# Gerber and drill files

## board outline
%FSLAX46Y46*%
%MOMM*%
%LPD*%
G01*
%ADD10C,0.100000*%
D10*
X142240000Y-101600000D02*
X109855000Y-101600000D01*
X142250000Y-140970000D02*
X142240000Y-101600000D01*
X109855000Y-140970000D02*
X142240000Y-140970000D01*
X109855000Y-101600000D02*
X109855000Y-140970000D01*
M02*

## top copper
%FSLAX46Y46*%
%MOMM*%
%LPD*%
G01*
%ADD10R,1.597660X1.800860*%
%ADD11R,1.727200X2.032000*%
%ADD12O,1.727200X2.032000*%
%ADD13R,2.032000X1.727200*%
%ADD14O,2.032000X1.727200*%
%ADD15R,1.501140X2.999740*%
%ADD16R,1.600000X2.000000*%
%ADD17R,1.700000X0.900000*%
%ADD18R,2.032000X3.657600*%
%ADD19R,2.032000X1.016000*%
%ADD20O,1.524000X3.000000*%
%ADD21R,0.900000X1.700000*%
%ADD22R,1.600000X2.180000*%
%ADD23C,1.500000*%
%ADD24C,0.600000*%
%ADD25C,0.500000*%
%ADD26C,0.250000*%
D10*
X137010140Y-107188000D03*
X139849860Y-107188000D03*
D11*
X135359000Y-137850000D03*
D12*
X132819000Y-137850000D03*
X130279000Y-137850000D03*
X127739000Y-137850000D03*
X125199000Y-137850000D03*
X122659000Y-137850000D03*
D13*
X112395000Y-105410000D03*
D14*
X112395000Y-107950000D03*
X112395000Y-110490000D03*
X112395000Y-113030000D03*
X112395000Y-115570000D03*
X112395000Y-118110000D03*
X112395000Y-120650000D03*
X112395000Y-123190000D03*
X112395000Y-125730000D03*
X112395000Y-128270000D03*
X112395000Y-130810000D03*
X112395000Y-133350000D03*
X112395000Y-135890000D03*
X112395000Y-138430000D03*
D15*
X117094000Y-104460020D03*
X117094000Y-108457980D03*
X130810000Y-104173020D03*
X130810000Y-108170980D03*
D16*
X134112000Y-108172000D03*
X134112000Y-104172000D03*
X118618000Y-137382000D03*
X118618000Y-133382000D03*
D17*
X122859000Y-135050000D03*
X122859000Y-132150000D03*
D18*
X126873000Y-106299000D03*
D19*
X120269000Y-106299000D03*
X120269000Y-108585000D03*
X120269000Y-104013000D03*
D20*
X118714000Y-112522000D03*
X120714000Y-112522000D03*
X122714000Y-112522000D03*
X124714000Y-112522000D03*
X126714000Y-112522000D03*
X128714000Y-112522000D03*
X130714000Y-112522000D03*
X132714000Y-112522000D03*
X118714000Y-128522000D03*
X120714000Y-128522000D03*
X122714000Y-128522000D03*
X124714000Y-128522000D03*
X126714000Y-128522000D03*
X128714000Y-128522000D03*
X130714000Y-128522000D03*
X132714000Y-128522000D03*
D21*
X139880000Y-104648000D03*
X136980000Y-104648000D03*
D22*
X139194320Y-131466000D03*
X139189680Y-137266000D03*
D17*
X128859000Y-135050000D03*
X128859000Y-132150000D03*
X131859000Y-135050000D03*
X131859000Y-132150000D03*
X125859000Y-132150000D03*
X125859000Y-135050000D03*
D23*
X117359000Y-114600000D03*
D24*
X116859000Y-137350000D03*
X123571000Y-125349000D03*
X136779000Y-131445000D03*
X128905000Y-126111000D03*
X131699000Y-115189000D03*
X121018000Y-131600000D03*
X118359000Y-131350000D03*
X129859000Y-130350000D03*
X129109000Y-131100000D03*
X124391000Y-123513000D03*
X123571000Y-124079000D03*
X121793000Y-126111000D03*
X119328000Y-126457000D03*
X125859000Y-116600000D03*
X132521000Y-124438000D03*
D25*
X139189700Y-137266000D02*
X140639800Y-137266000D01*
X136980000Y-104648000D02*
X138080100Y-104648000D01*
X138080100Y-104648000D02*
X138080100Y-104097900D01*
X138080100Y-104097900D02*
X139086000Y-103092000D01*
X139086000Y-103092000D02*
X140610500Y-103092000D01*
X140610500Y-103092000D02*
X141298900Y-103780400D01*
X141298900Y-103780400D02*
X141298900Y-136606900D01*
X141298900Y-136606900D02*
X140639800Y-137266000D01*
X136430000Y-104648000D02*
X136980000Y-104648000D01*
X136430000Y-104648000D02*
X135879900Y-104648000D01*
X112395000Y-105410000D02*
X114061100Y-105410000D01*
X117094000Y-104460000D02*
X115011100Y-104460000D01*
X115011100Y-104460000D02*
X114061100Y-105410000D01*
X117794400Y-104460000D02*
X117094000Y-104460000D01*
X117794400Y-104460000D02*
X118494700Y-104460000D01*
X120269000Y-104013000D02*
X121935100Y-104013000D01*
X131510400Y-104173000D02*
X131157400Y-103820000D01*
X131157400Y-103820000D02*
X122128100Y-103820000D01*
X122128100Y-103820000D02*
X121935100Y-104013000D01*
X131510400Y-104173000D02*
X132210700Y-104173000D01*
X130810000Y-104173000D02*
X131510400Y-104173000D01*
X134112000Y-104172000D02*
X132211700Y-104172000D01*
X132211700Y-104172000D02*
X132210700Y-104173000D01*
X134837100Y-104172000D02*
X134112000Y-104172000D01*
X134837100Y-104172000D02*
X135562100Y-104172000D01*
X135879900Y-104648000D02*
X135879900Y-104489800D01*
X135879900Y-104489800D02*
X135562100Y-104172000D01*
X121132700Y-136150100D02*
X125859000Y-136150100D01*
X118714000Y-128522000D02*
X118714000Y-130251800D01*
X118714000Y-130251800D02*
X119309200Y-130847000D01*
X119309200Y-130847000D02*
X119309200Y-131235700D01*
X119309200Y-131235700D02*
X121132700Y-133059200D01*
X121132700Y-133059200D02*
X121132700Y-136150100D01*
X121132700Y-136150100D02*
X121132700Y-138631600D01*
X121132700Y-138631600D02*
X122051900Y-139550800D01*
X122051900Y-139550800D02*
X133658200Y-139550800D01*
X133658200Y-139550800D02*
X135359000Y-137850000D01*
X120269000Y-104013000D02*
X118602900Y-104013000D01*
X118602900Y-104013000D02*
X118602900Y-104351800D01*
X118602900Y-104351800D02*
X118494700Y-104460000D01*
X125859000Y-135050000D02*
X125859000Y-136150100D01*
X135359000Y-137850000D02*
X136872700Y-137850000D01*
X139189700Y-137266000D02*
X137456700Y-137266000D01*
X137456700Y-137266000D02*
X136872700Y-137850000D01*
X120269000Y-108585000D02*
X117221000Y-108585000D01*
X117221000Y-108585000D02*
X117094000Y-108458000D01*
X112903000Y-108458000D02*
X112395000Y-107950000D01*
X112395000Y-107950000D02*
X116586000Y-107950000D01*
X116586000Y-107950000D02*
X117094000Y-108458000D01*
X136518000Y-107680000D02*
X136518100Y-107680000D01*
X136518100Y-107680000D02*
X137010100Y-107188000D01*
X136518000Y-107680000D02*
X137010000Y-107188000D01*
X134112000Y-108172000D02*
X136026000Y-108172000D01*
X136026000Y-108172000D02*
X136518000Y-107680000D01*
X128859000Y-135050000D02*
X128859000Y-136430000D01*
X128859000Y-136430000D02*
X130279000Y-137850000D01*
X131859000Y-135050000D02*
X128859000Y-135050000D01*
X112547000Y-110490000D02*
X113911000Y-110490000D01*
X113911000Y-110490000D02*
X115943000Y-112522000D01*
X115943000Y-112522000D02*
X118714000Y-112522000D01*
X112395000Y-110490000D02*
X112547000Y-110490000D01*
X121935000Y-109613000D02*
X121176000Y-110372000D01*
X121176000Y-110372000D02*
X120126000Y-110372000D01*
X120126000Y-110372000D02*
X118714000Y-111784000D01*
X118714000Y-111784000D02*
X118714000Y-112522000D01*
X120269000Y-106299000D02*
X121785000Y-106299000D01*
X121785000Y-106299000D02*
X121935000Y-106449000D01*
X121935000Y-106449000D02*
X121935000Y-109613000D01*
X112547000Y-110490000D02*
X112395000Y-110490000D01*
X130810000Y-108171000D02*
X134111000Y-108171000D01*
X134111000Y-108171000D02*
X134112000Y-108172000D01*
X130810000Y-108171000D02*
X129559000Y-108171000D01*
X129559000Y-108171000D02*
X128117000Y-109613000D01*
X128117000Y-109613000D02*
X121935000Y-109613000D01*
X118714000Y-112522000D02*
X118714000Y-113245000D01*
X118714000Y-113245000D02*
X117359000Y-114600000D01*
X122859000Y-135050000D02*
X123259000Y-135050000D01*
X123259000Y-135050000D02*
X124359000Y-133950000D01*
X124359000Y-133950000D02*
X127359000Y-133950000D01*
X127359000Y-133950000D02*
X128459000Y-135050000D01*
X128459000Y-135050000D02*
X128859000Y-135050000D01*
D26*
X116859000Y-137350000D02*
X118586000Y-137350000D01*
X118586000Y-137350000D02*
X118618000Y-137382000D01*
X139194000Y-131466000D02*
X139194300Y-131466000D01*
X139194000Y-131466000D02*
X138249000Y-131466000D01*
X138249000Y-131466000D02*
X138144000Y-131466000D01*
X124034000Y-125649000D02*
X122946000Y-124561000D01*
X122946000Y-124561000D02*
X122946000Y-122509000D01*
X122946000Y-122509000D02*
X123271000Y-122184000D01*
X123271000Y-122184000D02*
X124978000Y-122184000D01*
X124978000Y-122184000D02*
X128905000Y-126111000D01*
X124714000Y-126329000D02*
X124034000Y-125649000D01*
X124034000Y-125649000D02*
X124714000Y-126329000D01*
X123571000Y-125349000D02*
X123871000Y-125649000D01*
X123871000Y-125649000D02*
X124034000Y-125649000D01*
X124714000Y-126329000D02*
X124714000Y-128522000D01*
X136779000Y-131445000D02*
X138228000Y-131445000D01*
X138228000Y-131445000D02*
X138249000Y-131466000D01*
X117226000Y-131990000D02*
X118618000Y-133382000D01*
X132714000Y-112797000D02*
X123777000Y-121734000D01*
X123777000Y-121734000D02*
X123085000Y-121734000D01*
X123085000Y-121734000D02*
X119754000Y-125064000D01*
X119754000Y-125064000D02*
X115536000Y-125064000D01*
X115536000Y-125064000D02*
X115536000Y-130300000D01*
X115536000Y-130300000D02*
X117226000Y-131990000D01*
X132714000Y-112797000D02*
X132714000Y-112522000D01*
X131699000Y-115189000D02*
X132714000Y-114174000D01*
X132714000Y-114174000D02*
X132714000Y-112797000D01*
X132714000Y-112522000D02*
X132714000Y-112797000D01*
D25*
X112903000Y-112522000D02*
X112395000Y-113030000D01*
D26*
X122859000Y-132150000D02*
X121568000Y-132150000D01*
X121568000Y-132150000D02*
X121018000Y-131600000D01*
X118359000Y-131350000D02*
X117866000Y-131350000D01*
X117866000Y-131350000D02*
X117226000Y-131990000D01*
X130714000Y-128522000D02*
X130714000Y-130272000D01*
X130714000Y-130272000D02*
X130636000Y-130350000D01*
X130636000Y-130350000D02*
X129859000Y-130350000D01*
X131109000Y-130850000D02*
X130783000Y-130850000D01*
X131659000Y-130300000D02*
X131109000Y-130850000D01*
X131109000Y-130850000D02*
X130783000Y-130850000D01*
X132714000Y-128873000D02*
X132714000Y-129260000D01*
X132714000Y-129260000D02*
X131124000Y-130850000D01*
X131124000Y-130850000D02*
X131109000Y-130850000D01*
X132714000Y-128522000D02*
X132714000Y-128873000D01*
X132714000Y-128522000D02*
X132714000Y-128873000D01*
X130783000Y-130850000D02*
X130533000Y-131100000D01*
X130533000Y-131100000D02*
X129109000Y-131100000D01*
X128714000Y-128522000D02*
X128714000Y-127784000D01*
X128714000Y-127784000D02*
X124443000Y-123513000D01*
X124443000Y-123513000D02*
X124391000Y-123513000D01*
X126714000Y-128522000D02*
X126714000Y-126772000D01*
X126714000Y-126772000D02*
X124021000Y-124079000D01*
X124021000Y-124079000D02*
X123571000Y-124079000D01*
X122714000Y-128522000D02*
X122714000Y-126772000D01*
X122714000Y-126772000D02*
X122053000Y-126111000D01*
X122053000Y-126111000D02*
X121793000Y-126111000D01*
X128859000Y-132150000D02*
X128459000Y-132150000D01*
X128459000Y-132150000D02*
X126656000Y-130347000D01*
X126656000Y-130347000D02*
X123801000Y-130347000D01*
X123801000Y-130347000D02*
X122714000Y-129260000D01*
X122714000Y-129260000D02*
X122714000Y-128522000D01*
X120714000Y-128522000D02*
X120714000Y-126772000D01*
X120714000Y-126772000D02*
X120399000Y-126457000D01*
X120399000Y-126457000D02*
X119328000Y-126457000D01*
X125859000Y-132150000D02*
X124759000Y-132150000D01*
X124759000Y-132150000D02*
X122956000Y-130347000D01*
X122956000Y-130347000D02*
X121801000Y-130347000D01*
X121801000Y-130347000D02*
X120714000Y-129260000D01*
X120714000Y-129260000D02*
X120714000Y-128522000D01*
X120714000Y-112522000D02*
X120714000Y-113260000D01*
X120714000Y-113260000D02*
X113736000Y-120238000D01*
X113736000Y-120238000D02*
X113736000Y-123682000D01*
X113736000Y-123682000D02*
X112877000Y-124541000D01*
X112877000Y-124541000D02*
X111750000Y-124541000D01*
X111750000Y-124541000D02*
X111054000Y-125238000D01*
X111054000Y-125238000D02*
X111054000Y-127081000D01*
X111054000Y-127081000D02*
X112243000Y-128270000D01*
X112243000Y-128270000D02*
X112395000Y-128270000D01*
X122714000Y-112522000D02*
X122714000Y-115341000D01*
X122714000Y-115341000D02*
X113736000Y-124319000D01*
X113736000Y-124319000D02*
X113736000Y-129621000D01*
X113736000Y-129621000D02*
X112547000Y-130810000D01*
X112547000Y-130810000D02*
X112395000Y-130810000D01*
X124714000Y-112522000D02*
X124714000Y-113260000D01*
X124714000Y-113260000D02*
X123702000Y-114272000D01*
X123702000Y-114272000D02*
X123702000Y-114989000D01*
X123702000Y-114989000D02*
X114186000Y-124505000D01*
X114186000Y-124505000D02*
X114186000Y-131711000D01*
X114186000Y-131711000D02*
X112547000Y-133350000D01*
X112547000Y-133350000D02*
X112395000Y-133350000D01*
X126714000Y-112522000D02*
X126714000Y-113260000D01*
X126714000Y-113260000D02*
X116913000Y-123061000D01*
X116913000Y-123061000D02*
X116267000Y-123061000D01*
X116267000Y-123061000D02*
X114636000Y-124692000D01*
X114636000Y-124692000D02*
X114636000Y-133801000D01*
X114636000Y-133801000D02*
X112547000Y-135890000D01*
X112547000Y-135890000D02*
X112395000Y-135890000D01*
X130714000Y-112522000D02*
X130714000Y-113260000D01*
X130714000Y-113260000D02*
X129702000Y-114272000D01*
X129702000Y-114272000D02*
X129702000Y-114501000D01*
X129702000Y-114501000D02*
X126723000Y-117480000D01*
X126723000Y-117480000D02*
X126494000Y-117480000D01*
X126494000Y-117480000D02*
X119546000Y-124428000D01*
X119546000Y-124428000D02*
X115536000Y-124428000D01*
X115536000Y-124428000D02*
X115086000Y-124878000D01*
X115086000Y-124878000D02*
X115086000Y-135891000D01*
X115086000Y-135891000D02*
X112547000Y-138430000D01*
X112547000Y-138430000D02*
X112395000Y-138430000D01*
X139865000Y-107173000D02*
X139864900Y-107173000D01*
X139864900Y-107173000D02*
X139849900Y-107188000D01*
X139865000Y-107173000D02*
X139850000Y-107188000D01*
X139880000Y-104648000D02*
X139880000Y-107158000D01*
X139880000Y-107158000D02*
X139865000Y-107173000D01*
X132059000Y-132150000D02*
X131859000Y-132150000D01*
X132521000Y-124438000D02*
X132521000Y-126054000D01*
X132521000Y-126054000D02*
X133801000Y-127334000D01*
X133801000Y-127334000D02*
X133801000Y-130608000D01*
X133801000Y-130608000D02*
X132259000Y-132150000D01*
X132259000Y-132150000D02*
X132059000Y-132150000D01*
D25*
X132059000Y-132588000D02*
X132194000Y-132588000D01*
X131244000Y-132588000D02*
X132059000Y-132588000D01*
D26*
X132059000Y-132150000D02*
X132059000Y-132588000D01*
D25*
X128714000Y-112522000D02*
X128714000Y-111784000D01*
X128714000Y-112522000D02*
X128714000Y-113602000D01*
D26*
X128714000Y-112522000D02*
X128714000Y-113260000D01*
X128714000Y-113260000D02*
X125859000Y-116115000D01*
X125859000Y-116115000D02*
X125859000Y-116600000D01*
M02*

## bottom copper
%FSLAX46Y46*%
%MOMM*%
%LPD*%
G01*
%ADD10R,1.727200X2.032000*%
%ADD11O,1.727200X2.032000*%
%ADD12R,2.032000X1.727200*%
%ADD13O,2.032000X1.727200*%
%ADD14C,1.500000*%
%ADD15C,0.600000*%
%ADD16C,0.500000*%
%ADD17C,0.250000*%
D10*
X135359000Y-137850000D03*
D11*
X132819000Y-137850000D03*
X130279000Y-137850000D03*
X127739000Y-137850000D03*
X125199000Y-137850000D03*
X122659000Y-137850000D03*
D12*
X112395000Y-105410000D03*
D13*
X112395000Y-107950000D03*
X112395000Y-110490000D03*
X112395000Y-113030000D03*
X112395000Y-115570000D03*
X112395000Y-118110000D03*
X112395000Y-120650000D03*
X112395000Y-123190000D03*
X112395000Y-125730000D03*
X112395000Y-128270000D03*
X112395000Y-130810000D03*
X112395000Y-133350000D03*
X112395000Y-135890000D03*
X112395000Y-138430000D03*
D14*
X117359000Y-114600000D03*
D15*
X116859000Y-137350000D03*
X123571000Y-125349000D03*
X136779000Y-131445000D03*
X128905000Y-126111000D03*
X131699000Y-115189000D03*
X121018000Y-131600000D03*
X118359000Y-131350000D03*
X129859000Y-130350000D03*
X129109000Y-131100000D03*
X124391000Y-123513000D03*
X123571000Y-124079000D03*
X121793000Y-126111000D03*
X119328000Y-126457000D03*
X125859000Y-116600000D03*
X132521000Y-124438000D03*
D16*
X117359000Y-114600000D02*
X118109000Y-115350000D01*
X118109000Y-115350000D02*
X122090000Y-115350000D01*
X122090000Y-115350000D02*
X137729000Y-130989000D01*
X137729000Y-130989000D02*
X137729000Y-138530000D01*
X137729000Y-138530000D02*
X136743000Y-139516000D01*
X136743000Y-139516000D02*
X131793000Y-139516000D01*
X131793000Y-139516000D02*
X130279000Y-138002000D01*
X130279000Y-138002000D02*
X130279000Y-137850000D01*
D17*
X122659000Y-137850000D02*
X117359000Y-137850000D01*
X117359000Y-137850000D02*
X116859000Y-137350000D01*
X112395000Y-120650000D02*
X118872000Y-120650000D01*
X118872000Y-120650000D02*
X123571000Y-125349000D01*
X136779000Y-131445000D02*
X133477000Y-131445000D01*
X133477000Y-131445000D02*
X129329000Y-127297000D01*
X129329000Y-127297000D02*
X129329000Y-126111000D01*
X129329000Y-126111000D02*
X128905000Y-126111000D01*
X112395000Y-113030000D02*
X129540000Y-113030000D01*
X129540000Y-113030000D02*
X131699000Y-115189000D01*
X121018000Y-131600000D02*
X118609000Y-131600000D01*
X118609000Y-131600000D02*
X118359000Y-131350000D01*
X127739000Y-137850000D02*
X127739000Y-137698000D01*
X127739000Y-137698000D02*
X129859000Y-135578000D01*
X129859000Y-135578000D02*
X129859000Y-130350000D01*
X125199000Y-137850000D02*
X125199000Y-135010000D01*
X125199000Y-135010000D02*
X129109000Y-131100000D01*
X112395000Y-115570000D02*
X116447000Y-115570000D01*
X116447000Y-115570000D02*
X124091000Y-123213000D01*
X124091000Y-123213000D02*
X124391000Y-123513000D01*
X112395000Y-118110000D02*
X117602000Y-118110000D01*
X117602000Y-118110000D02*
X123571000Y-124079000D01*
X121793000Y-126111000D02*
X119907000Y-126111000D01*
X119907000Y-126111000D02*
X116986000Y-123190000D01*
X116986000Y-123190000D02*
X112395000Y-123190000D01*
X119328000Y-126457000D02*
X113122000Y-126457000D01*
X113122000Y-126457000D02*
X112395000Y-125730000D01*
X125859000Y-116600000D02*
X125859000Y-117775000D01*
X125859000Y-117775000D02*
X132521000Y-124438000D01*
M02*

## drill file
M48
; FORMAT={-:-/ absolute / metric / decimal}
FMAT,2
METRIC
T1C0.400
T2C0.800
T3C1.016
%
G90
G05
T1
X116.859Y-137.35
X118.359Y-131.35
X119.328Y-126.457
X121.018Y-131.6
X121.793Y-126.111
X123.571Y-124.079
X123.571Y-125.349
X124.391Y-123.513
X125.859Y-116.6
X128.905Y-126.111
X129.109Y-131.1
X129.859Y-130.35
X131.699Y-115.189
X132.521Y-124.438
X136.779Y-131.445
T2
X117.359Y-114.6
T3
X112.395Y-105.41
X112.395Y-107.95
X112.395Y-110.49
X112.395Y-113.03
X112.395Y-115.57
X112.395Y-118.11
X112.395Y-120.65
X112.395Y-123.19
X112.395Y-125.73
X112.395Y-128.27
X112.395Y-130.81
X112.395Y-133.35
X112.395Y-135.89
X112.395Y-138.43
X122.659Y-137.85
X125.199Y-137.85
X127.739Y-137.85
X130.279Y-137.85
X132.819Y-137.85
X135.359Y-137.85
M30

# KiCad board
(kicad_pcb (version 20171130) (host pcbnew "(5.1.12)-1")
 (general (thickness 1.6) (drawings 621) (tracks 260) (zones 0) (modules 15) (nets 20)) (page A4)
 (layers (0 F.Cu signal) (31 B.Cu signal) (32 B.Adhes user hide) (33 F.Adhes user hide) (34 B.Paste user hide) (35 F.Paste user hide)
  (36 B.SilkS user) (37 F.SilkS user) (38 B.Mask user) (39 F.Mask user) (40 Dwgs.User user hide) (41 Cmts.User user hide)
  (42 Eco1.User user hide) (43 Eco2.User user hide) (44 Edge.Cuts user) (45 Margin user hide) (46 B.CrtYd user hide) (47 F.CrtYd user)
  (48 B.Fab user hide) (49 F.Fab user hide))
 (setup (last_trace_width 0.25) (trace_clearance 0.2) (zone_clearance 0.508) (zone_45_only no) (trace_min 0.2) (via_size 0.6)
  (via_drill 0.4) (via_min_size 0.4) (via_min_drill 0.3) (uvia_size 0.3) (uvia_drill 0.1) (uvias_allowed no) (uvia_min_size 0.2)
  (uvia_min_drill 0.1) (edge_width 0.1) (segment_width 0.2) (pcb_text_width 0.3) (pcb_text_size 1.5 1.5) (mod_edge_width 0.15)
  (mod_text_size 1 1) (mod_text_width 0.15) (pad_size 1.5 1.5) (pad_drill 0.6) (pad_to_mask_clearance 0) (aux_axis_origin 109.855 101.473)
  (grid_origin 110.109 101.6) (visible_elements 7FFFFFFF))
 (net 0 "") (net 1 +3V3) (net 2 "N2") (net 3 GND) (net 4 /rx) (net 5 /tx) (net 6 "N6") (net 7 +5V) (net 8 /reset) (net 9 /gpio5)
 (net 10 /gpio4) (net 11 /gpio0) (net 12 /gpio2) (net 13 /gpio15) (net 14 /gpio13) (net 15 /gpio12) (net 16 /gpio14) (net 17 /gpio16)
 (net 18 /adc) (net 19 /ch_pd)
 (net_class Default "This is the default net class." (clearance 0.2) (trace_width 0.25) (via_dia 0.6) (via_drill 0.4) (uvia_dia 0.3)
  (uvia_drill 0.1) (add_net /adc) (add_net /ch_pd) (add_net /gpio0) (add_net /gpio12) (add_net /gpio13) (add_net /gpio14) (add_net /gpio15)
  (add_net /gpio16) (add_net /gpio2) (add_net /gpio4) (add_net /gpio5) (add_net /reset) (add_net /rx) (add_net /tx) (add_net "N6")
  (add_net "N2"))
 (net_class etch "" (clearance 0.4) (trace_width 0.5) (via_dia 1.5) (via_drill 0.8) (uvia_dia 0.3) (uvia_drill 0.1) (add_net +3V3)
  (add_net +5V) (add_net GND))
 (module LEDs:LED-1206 (layer F.Cu) (at 138.43 107.188 180)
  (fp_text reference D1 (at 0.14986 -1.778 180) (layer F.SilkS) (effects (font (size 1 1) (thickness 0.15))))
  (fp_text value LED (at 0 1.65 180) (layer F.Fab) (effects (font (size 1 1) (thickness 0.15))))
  (pad 2 smd rect (at 1.41986 0) (size 1.59766 1.80086) (layers F.Cu F.Paste F.Mask) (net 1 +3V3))
  (pad 1 smd rect (at -1.41986 0) (size 1.59766 1.80086) (layers F.Cu F.Paste F.Mask) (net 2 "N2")))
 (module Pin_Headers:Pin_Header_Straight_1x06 (layer F.Cu) (at 135.359 137.85 270)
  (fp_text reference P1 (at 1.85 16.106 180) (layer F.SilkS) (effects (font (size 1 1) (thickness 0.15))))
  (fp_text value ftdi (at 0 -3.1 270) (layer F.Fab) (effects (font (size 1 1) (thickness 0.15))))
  (pad 1 thru_hole rect (at 0 0 270) (size 2.032 1.7272) (drill 1.016) (layers *.Cu *.Mask F.SilkS) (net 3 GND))
  (pad 2 thru_hole oval (at 0 2.54 270) (size 2.032 1.7272) (drill 1.016) (layers *.Cu *.Mask F.SilkS))
  (pad 3 thru_hole oval (at 0 5.08 270) (size 2.032 1.7272) (drill 1.016) (layers *.Cu *.Mask F.SilkS) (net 1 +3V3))
  (pad 4 thru_hole oval (at 0 7.62 270) (size 2.032 1.7272) (drill 1.016) (layers *.Cu *.Mask F.SilkS) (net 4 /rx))
  (pad 5 thru_hole oval (at 0 10.16 270) (size 2.032 1.7272) (drill 1.016) (layers *.Cu *.Mask F.SilkS) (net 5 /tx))
  (pad 6 thru_hole oval (at 0 12.7 270) (size 2.032 1.7272) (drill 1.016) (layers *.Cu *.Mask F.SilkS) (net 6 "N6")))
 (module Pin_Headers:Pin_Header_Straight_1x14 (layer B.Cu) (at 112.395 105.41 180)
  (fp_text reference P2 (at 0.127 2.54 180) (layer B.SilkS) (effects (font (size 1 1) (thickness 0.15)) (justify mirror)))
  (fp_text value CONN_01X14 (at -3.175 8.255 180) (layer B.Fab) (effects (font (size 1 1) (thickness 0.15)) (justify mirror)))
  (pad 1 thru_hole rect (at 0 0 180) (size 2.032 1.7272) (drill 1.016) (layers *.Cu *.Mask B.SilkS) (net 3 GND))
  (pad 2 thru_hole oval (at 0 -2.54 180) (size 2.032 1.7272) (drill 1.016) (layers *.Cu *.Mask B.SilkS) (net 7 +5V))
  (pad 3 thru_hole oval (at 0 -5.08 180) (size 2.032 1.7272) (drill 1.016) (layers *.Cu *.Mask B.SilkS) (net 1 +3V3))
  (pad 4 thru_hole oval (at 0 -7.62 180) (size 2.032 1.7272) (drill 1.016) (layers *.Cu *.Mask B.SilkS) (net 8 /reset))
  (pad 5 thru_hole oval (at 0 -10.16 180) (size 2.032 1.7272) (drill 1.016) (layers *.Cu *.Mask B.SilkS) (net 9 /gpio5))
  (pad 6 thru_hole oval (at 0 -12.7 180) (size 2.032 1.7272) (drill 1.016) (layers *.Cu *.Mask B.SilkS) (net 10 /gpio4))
  (pad 7 thru_hole oval (at 0 -15.24 180) (size 2.032 1.7272) (drill 1.016) (layers *.Cu *.Mask B.SilkS) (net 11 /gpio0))
  (pad 8 thru_hole oval (at 0 -17.78 180) (size 2.032 1.7272) (drill 1.016) (layers *.Cu *.Mask B.SilkS) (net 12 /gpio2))
  (pad 9 thru_hole oval (at 0 -20.32 180) (size 2.032 1.7272) (drill 1.016) (layers *.Cu *.Mask B.SilkS) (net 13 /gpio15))
  (pad 10 thru_hole oval (at 0 -22.86 180) (size 2.032 1.7272) (drill 1.016) (layers *.Cu *.Mask B.SilkS) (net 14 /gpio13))
  (pad 11 thru_hole oval (at 0 -25.4 180) (size 2.032 1.7272) (drill 1.016) (layers *.Cu *.Mask B.SilkS) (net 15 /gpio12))
  (pad 12 thru_hole oval (at 0 -27.94 180) (size 2.032 1.7272) (drill 1.016) (layers *.Cu *.Mask B.SilkS) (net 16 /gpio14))
  (pad 13 thru_hole oval (at 0 -30.48 180) (size 2.032 1.7272) (drill 1.016) (layers *.Cu *.Mask B.SilkS) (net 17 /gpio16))
  (pad 14 thru_hole oval (at 0 -33.02 180) (size 2.032 1.7272) (drill 1.016) (layers *.Cu *.Mask B.SilkS) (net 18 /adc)))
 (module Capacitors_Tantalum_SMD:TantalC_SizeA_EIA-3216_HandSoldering (layer F.Cu) (at 117.094 106.459 90)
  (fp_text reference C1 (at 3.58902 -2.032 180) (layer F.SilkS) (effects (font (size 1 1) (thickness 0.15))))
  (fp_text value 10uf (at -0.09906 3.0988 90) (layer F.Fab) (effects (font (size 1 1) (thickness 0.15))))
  (pad 2 smd rect (at 1.99898 0 90) (size 2.99974 1.50114) (layers F.Cu F.Paste F.Mask) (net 3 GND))
  (pad 1 smd rect (at -1.99898 0 90) (size 2.99974 1.50114) (layers F.Cu F.Paste F.Mask) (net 7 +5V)))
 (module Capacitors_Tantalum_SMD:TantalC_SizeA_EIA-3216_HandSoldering (layer F.Cu) (at 130.81 106.172 90)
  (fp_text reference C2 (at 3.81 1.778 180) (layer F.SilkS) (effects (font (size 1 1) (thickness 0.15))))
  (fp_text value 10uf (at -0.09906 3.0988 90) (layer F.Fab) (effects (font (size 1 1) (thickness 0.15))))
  (pad 2 smd rect (at 1.99898 0 90) (size 2.99974 1.50114) (layers F.Cu F.Paste F.Mask) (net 3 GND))
  (pad 1 smd rect (at -1.99898 0 90) (size 2.99974 1.50114) (layers F.Cu F.Paste F.Mask) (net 1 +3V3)))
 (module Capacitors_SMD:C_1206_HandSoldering (layer F.Cu) (at 134.112 106.172 90)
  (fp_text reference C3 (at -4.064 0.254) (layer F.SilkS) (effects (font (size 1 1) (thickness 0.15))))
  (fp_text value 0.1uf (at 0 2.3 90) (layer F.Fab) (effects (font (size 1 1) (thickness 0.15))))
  (pad 1 smd rect (at -2 0 90) (size 2 1.6) (layers F.Cu F.Paste F.Mask) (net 1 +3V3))
  (pad 2 smd rect (at 2 0 90) (size 2 1.6) (layers F.Cu F.Paste F.Mask) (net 3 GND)))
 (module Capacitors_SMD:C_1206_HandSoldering (layer F.Cu) (at 118.618 135.382 90)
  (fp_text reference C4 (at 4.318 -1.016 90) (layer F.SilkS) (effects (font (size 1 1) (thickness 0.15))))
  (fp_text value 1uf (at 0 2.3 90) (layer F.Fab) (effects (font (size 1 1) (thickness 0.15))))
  (pad 1 smd rect (at -2 0 90) (size 2 1.6) (layers F.Cu F.Paste F.Mask) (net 6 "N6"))
  (pad 2 smd rect (at 2 0 90) (size 2 1.6) (layers F.Cu F.Paste F.Mask) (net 8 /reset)))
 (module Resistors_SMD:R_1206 (layer F.Cu) (at 122.859 133.6 90)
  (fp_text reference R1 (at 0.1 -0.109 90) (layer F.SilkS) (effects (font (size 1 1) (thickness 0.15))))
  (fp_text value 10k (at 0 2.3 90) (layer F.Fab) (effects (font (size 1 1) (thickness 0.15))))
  (pad 1 smd rect (at -1.45 0 90) (size 0.9 1.7) (layers F.Cu F.Paste F.Mask) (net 1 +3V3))
  (pad 2 smd rect (at 1.45 0 90) (size 0.9 1.7) (layers F.Cu F.Paste F.Mask) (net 8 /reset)))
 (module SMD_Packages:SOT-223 (layer F.Cu) (at 123.571 106.299 270)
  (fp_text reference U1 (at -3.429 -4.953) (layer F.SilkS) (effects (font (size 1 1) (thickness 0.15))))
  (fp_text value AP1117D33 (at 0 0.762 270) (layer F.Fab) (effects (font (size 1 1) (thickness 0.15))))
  (pad 4 smd rect (at 0 -3.302 270) (size 3.6576 2.032) (layers F.Cu F.Paste F.Mask))
  (pad 2 smd rect (at 0 3.302 270) (size 1.016 2.032) (layers F.Cu F.Paste F.Mask) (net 1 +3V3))
  (pad 3 smd rect (at 2.286 3.302 270) (size 1.016 2.032) (layers F.Cu F.Paste F.Mask) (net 7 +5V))
  (pad 1 smd rect (at -2.286 3.302 270) (size 1.016 2.032) (layers F.Cu F.Paste F.Mask) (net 3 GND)))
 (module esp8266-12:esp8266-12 (layer F.Cu) (at 118.714 112.622)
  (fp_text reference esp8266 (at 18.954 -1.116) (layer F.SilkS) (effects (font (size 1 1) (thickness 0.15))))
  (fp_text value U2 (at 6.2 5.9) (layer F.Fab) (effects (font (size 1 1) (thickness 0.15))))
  (pad 8 smd oval (at 0 -0.1) (size 1.524 3) (layers F.Cu F.Paste F.Mask) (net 1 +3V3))
  (pad 7 smd oval (at 2 -0.1) (size 1.524 3) (layers F.Cu F.Paste F.Mask) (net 14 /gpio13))
  (pad 6 smd oval (at 4 -0.1) (size 1.524 3) (layers F.Cu F.Paste F.Mask) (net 15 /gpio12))
  (pad 5 smd oval (at 6 -0.1) (size 1.524 3) (layers F.Cu F.Paste F.Mask) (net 16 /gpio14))
  (pad 4 smd oval (at 8 -0.1) (size 1.524 3) (layers F.Cu F.Paste F.Mask) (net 17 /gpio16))
  (pad 3 smd oval (at 10 -0.1) (size 1.524 3) (layers F.Cu F.Paste F.Mask) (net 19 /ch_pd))
  (pad 2 smd oval (at 12 -0.1) (size 1.524 3) (layers F.Cu F.Paste F.Mask) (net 18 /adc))
  (pad 1 smd oval (at 14 -0.1) (size 1.524 3) (layers F.Cu F.Paste F.Mask) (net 8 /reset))
  (pad 9 smd oval (at 0 15.9) (size 1.524 3) (layers F.Cu F.Paste F.Mask) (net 3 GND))
  (pad 10 smd oval (at 2 15.9) (size 1.524 3) (layers F.Cu F.Paste F.Mask) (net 13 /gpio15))
  (pad 11 smd oval (at 4 15.9) (size 1.524 3) (layers F.Cu F.Paste F.Mask) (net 12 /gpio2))
  (pad 12 smd oval (at 6 15.9) (size 1.524 3) (layers F.Cu F.Paste F.Mask) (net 11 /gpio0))
  (pad 13 smd oval (at 8 15.9) (size 1.524 3) (layers F.Cu F.Paste F.Mask) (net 10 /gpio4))
  (pad 14 smd oval (at 10 15.9) (size 1.524 3) (layers F.Cu F.Paste F.Mask) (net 9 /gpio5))
  (pad 15 smd oval (at 12 15.9) (size 1.524 3) (layers F.Cu F.Paste F.Mask) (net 4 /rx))
  (pad 16 smd oval (at 14 15.9) (size 1.524 3) (layers F.Cu F.Paste F.Mask) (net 5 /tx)))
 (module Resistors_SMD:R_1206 (layer F.Cu) (at 138.43 104.648 180)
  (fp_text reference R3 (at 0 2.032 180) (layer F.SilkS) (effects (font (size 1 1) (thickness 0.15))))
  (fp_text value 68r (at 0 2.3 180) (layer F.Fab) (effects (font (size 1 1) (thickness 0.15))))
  (pad 1 smd rect (at -1.45 0 180) (size 0.9 1.7) (layers F.Cu F.Paste F.Mask) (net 2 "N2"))
  (pad 2 smd rect (at 1.45 0 180) (size 0.9 1.7) (layers F.Cu F.Paste F.Mask) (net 3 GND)))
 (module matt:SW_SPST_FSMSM (layer F.Cu) (at 139.192 134.366 270)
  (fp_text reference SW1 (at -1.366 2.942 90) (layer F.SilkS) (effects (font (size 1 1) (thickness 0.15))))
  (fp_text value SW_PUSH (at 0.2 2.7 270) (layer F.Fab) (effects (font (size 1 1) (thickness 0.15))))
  (pad 1 smd rect (at -2.9 -0.00232 270) (size 2.18 1.6) (layers F.Cu F.Paste F.Mask) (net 11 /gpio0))
  (pad 2 smd rect (at 2.9 0.00232 270) (size 2.18 1.6) (layers F.Cu F.Paste F.Mask) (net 3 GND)))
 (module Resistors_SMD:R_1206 (layer F.Cu) (at 128.859 133.6 90)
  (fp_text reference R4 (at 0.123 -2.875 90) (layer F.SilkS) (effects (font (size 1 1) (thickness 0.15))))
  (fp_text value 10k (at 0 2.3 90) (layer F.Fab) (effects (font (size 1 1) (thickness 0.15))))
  (pad 1 smd rect (at -1.45 0 90) (size 0.9 1.7) (layers F.Cu F.Paste F.Mask) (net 1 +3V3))
  (pad 2 smd rect (at 1.45 0 90) (size 0.9 1.7) (layers F.Cu F.Paste F.Mask) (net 12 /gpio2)))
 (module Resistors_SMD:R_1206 (layer F.Cu) (at 131.859 133.6 90)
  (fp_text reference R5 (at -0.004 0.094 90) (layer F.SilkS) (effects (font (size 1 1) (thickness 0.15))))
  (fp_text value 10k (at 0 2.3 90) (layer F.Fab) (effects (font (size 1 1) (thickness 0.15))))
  (pad 1 smd rect (at -1.45 0 90) (size 0.9 1.7) (layers F.Cu F.Paste F.Mask) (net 1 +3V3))
  (pad 2 smd rect (at 1.45 0 90) (size 0.9 1.7) (layers F.Cu F.Paste F.Mask) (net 19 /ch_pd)))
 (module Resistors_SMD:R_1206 (layer F.Cu) (at 125.859 133.6 270)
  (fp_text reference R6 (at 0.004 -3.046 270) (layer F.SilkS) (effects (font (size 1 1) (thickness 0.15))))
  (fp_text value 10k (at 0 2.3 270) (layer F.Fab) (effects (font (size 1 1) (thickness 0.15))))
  (pad 1 smd rect (at -1.45 0 270) (size 0.9 1.7) (layers F.Cu F.Paste F.Mask) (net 13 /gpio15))
  (pad 2 smd rect (at 1.45 0 270) (size 0.9 1.7) (layers F.Cu F.Paste F.Mask) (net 3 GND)))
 (gr_line (start 142.24 101.6) (end 109.855 101.6) (layer Edge.Cuts) (width 0.1))
 (gr_line (start 142.25 140.97) (end 142.24 101.6) (layer Edge.Cuts) (width 0.1))
 (gr_line (start 109.855 140.97) (end 142.24 140.97) (layer Edge.Cuts) (width 0.1))
 (gr_line (start 109.855 101.6) (end 109.855 140.97) (layer Edge.Cuts) (width 0.1))
 (segment (start 139.1897 137.266) (end 140.6398 137.266) (width 0.5) (layer F.Cu) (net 3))
 (segment (start 136.98 104.648) (end 138.0801 104.648) (width 0.5) (layer F.Cu) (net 3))
 (segment (start 138.0801 104.648) (end 138.0801 104.0979) (width 0.5) (layer F.Cu) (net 3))
 (segment (start 138.0801 104.0979) (end 139.086 103.092) (width 0.5) (layer F.Cu) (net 3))
 (segment (start 139.086 103.092) (end 140.6105 103.092) (width 0.5) (layer F.Cu) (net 3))
 (segment (start 140.6105 103.092) (end 141.2989 103.7804) (width 0.5) (layer F.Cu) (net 3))
 (segment (start 141.2989 103.7804) (end 141.2989 136.6069) (width 0.5) (layer F.Cu) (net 3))
 (segment (start 141.2989 136.6069) (end 140.6398 137.266) (width 0.5) (layer F.Cu) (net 3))
 (segment (start 136.43 104.648) (end 136.98 104.648) (width 0.5) (layer F.Cu) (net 3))
 (segment (start 136.43 104.648) (end 135.8799 104.648) (width 0.5) (layer F.Cu) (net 3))
 (segment (start 112.395 105.41) (end 114.0611 105.41) (width 0.5) (layer F.Cu) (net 3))
 (segment (start 117.094 104.46) (end 115.0111 104.46) (width 0.5) (layer F.Cu) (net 3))
 (segment (start 115.0111 104.46) (end 114.0611 105.41) (width 0.5) (layer F.Cu) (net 3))
 (segment (start 117.7944 104.46) (end 117.094 104.46) (width 0.5) (layer F.Cu) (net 3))
 (segment (start 117.7944 104.46) (end 118.4947 104.46) (width 0.5) (layer F.Cu) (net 3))
 (segment (start 120.269 104.013) (end 121.9351 104.013) (width 0.5) (layer F.Cu) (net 3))
 (segment (start 131.5104 104.173) (end 131.1574 103.82) (width 0.5) (layer F.Cu) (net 3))
 (segment (start 131.1574 103.82) (end 122.1281 103.82) (width 0.5) (layer F.Cu) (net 3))
 (segment (start 122.1281 103.82) (end 121.9351 104.013) (width 0.5) (layer F.Cu) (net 3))
 (segment (start 131.5104 104.173) (end 132.2107 104.173) (width 0.5) (layer F.Cu) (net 3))
 (segment (start 130.81 104.173) (end 131.5104 104.173) (width 0.5) (layer F.Cu) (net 3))
 (segment (start 134.112 104.172) (end 132.2117 104.172) (width 0.5) (layer F.Cu) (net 3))
 (segment (start 132.2117 104.172) (end 132.2107 104.173) (width 0.5) (layer F.Cu) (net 3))
 (segment (start 134.8371 104.172) (end 134.112 104.172) (width 0.5) (layer F.Cu) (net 3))
 (segment (start 134.8371 104.172) (end 135.5621 104.172) (width 0.5) (layer F.Cu) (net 3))
 (segment (start 135.8799 104.648) (end 135.8799 104.4898) (width 0.5) (layer F.Cu) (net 3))
 (segment (start 135.8799 104.4898) (end 135.5621 104.172) (width 0.5) (layer F.Cu) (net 3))
 (segment (start 121.1327 136.1501) (end 125.859 136.1501) (width 0.5) (layer F.Cu) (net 3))
 (segment (start 118.714 128.522) (end 118.714 130.2518) (width 0.5) (layer F.Cu) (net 3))
 (segment (start 118.714 130.2518) (end 119.3092 130.847) (width 0.5) (layer F.Cu) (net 3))
 (segment (start 119.3092 130.847) (end 119.3092 131.2357) (width 0.5) (layer F.Cu) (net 3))
 (segment (start 119.3092 131.2357) (end 121.1327 133.0592) (width 0.5) (layer F.Cu) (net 3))
 (segment (start 121.1327 133.0592) (end 121.1327 136.1501) (width 0.5) (layer F.Cu) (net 3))
 (segment (start 121.1327 136.1501) (end 121.1327 138.6316) (width 0.5) (layer F.Cu) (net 3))
 (segment (start 121.1327 138.6316) (end 122.0519 139.5508) (width 0.5) (layer F.Cu) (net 3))
 (segment (start 122.0519 139.5508) (end 133.6582 139.5508) (width 0.5) (layer F.Cu) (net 3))
 (segment (start 133.6582 139.5508) (end 135.359 137.85) (width 0.5) (layer F.Cu) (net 3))
 (segment (start 120.269 104.013) (end 118.6029 104.013) (width 0.5) (layer F.Cu) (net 3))
 (segment (start 118.6029 104.013) (end 118.6029 104.3518) (width 0.5) (layer F.Cu) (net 3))
 (segment (start 118.6029 104.3518) (end 118.4947 104.46) (width 0.5) (layer F.Cu) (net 3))
 (segment (start 125.859 135.05) (end 125.859 136.1501) (width 0.5) (layer F.Cu) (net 3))
 (segment (start 135.359 137.85) (end 136.8727 137.85) (width 0.5) (layer F.Cu) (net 3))
 (segment (start 139.1897 137.266) (end 137.4567 137.266) (width 0.5) (layer F.Cu) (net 3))
 (segment (start 137.4567 137.266) (end 136.8727 137.85) (width 0.5) (layer F.Cu) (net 3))
 (segment (start 120.269 108.585) (end 117.221 108.585) (width 0.5) (layer F.Cu) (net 7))
 (segment (start 117.221 108.585) (end 117.094 108.458) (width 0.5) (layer F.Cu) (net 7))
 (segment (start 112.903 108.458) (end 112.395 107.95) (width 0.5) (layer F.Cu) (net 7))
 (segment (start 112.395 107.95) (end 116.586 107.95) (width 0.5) (layer F.Cu) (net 7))
 (segment (start 116.586 107.95) (end 117.094 108.458) (width 0.5) (layer F.Cu) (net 7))
 (segment (start 136.518 107.68) (end 136.5181 107.68) (width 0.5) (layer F.Cu) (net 1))
 (segment (start 136.5181 107.68) (end 137.0101 107.188) (width 0.5) (layer F.Cu) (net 1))
 (segment (start 136.518 107.68) (end 137.01 107.188) (width 0.5) (layer F.Cu) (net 1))
 (segment (start 134.112 108.172) (end 136.026 108.172) (width 0.5) (layer F.Cu) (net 1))
 (segment (start 136.026 108.172) (end 136.518 107.68) (width 0.5) (layer F.Cu) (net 1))
 (segment (start 128.859 135.05) (end 128.859 136.43) (width 0.5) (layer F.Cu) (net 1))
 (segment (start 128.859 136.43) (end 130.279 137.85) (width 0.5) (layer F.Cu) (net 1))
 (segment (start 131.859 135.05) (end 128.859 135.05) (width 0.5) (layer F.Cu) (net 1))
 (segment (start 112.547 110.49) (end 113.911 110.49) (width 0.5) (layer F.Cu) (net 1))
 (segment (start 113.911 110.49) (end 115.943 112.522) (width 0.5) (layer F.Cu) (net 1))
 (segment (start 115.943 112.522) (end 118.714 112.522) (width 0.5) (layer F.Cu) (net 1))
 (segment (start 112.395 110.49) (end 112.547 110.49) (width 0.5) (layer F.Cu) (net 1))
 (segment (start 121.935 109.613) (end 121.176 110.372) (width 0.5) (layer F.Cu) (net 1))
 (segment (start 121.176 110.372) (end 120.126 110.372) (width 0.5) (layer F.Cu) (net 1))
 (segment (start 120.126 110.372) (end 118.714 111.784) (width 0.5) (layer F.Cu) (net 1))
 (segment (start 118.714 111.784) (end 118.714 112.522) (width 0.5) (layer F.Cu) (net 1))
 (segment (start 120.269 106.299) (end 121.785 106.299) (width 0.5) (layer F.Cu) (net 1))
 (segment (start 121.785 106.299) (end 121.935 106.449) (width 0.5) (layer F.Cu) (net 1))
 (segment (start 121.935 106.449) (end 121.935 109.613) (width 0.5) (layer F.Cu) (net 1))
 (segment (start 112.547 110.49) (end 112.395 110.49) (width 0.5) (layer F.Cu) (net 1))
 (segment (start 130.81 108.171) (end 134.111 108.171) (width 0.5) (layer F.Cu) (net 1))
 (segment (start 134.111 108.171) (end 134.112 108.172) (width 0.5) (layer F.Cu) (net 1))
 (segment (start 130.81 108.171) (end 129.559 108.171) (width 0.5) (layer F.Cu) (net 1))
 (segment (start 129.559 108.171) (end 128.117 109.613) (width 0.5) (layer F.Cu) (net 1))
 (segment (start 128.117 109.613) (end 121.935 109.613) (width 0.5) (layer F.Cu) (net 1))
 (segment (start 118.714 112.522) (end 118.714 113.245) (width 0.5) (layer F.Cu) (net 1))
 (segment (start 118.714 113.245) (end 117.359 114.6) (width 0.5) (layer F.Cu) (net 1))
 (segment (start 117.359 114.6) (end 118.109 115.35) (width 0.5) (layer B.Cu) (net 1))
 (segment (start 118.109 115.35) (end 122.09 115.35) (width 0.5) (layer B.Cu) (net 1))
 (segment (start 122.09 115.35) (end 137.729 130.989) (width 0.5) (layer B.Cu) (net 1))
 (segment (start 137.729 130.989) (end 137.729 138.53) (width 0.5) (layer B.Cu) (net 1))
 (segment (start 137.729 138.53) (end 136.743 139.516) (width 0.5) (layer B.Cu) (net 1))
 (segment (start 136.743 139.516) (end 131.793 139.516) (width 0.5) (layer B.Cu) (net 1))
 (segment (start 131.793 139.516) (end 130.279 138.002) (width 0.5) (layer B.Cu) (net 1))
 (segment (start 130.279 138.002) (end 130.279 137.85) (width 0.5) (layer B.Cu) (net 1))
 (segment (start 122.859 135.05) (end 123.259 135.05) (width 0.5) (layer F.Cu) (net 1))
 (segment (start 123.259 135.05) (end 124.359 133.95) (width 0.5) (layer F.Cu) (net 1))
 (segment (start 124.359 133.95) (end 127.359 133.95) (width 0.5) (layer F.Cu) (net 1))
 (segment (start 127.359 133.95) (end 128.459 135.05) (width 0.5) (layer F.Cu) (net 1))
 (segment (start 128.459 135.05) (end 128.859 135.05) (width 0.5) (layer F.Cu) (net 1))
 (via (at 117.359 114.6) (size 1.5) (drill 0.8) (layers F.Cu B.Cu) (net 1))
 (segment (start 122.659 137.85) (end 117.359 137.85) (width 0.25) (layer B.Cu) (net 6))
 (segment (start 117.359 137.85) (end 116.859 137.35) (width 0.25) (layer B.Cu) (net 6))
 (segment (start 116.859 137.35) (end 118.586 137.35) (width 0.25) (layer F.Cu) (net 6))
 (segment (start 118.586 137.35) (end 118.618 137.382) (width 0.25) (layer F.Cu) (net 6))
 (via (at 116.859 137.35) (size 0.6) (layers F.Cu B.Cu) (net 6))
 (segment (start 139.194 131.466) (end 139.1943 131.466) (width 0.25) (layer F.Cu) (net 11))
 (segment (start 139.194 131.466) (end 138.249 131.466) (width 0.25) (layer F.Cu) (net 11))
 (segment (start 138.249 131.466) (end 138.144 131.466) (width 0.25) (layer F.Cu) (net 11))
 (segment (start 124.034 125.649) (end 122.946 124.561) (width 0.25) (layer F.Cu) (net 11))
 (segment (start 122.946 124.561) (end 122.946 122.509) (width 0.25) (layer F.Cu) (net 11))
 (segment (start 122.946 122.509) (end 123.271 122.184) (width 0.25) (layer F.Cu) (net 11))
 (segment (start 123.271 122.184) (end 124.978 122.184) (width 0.25) (layer F.Cu) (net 11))
 (segment (start 124.978 122.184) (end 128.905 126.111) (width 0.25) (layer F.Cu) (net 11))
 (segment (start 124.714 126.329) (end 124.034 125.649) (width 0.25) (layer F.Cu) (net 11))
 (segment (start 124.034 125.649) (end 124.714 126.329) (width 0.25) (layer F.Cu) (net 11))
 (segment (start 123.571 125.349) (end 123.871 125.649) (width 0.25) (layer F.Cu) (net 11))
 (segment (start 123.871 125.649) (end 124.034 125.649) (width 0.25) (layer F.Cu) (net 11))
 (segment (start 124.714 126.329) (end 124.714 128.522) (width 0.25) (layer F.Cu) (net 11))
 (segment (start 112.395 120.65) (end 118.872 120.65) (width 0.25) (layer B.Cu) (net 11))
 (segment (start 118.872 120.65) (end 123.571 125.349) (width 0.25) (layer B.Cu) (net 11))
 (segment (start 136.779 131.445) (end 138.228 131.445) (width 0.25) (layer F.Cu) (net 11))
 (segment (start 138.228 131.445) (end 138.249 131.466) (width 0.25) (layer F.Cu) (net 11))
 (segment (start 136.779 131.445) (end 133.477 131.445) (width 0.25) (layer B.Cu) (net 11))
 (segment (start 133.477 131.445) (end 129.329 127.297) (width 0.25) (layer B.Cu) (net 11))
 (segment (start 129.329 127.297) (end 129.329 126.111) (width 0.25) (layer B.Cu) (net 11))
 (segment (start 129.329 126.111) (end 128.905 126.111) (width 0.25) (layer B.Cu) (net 11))
 (via (at 123.571 125.349) (size 0.6) (layers F.Cu B.Cu) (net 11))
 (via (at 136.779 131.445) (size 0.6) (layers F.Cu B.Cu) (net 11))
 (via (at 128.905 126.111) (size 0.6) (layers F.Cu B.Cu) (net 11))
 (segment (start 117.226 131.99) (end 118.618 133.382) (width 0.25) (layer F.Cu) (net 8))
 (segment (start 132.714 112.797) (end 123.777 121.734) (width 0.25) (layer F.Cu) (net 8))
 (segment (start 123.777 121.734) (end 123.085 121.734) (width 0.25) (layer F.Cu) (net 8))
 (segment (start 123.085 121.734) (end 119.754 125.064) (width 0.25) (layer F.Cu) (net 8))
 (segment (start 119.754 125.064) (end 115.536 125.064) (width 0.25) (layer F.Cu) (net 8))
 (segment (start 115.536 125.064) (end 115.536 130.3) (width 0.25) (layer F.Cu) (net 8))
 (segment (start 115.536 130.3) (end 117.226 131.99) (width 0.25) (layer F.Cu) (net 8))
 (segment (start 132.714 112.797) (end 132.714 112.522) (width 0.25) (layer F.Cu) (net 8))
 (segment (start 131.699 115.189) (end 132.714 114.174) (width 0.25) (layer F.Cu) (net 8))
 (segment (start 132.714 114.174) (end 132.714 112.797) (width 0.25) (layer F.Cu) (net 8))
 (segment (start 132.714 112.522) (end 132.714 112.797) (width 0.25) (layer F.Cu) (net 8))
 (segment (start 112.903 112.522) (end 112.395 113.03) (width 0.5) (layer F.Cu) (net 8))
 (segment (start 112.395 113.03) (end 129.54 113.03) (width 0.25) (layer B.Cu) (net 8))
 (segment (start 129.54 113.03) (end 131.699 115.189) (width 0.25) (layer B.Cu) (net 8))
 (segment (start 122.859 132.15) (end 121.568 132.15) (width 0.25) (layer F.Cu) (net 8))
 (segment (start 121.568 132.15) (end 121.018 131.6) (width 0.25) (layer F.Cu) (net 8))
 (segment (start 121.018 131.6) (end 118.609 131.6) (width 0.25) (layer B.Cu) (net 8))
 (segment (start 118.609 131.6) (end 118.359 131.35) (width 0.25) (layer B.Cu) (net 8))
 (segment (start 118.359 131.35) (end 117.866 131.35) (width 0.25) (layer F.Cu) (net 8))
 (segment (start 117.866 131.35) (end 117.226 131.99) (width 0.25) (layer F.Cu) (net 8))
 (via (at 131.699 115.189) (size 0.6) (layers F.Cu B.Cu) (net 8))
 (via (at 121.018 131.6) (size 0.6) (layers F.Cu B.Cu) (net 8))
 (via (at 118.359 131.35) (size 0.6) (layers F.Cu B.Cu) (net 8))
 (segment (start 130.714 128.522) (end 130.714 130.272) (width 0.25) (layer F.Cu) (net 4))
 (segment (start 130.714 130.272) (end 130.636 130.35) (width 0.25) (layer F.Cu) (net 4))
 (segment (start 130.636 130.35) (end 129.859 130.35) (width 0.25) (layer F.Cu) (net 4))
 (segment (start 127.739 137.85) (end 127.739 137.698) (width 0.25) (layer B.Cu) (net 4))
 (segment (start 127.739 137.698) (end 129.859 135.578) (width 0.25) (layer B.Cu) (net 4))
 (segment (start 129.859 135.578) (end 129.859 130.35) (width 0.25) (layer B.Cu) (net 4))
 (via (at 129.859 130.35) (size 0.6) (layers F.Cu B.Cu) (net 4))
 (segment (start 131.109 130.85) (end 130.783 130.85) (width 0.25) (layer F.Cu) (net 5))
 (segment (start 131.659 130.3) (end 131.109 130.85) (width 0.25) (layer F.Cu) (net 5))
 (segment (start 131.109 130.85) (end 130.783 130.85) (width 0.25) (layer F.Cu) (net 5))
 (segment (start 132.714 128.873) (end 132.714 129.26) (width 0.25) (layer F.Cu) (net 5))
 (segment (start 132.714 129.26) (end 131.124 130.85) (width 0.25) (layer F.Cu) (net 5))
 (segment (start 131.124 130.85) (end 131.109 130.85) (width 0.25) (layer F.Cu) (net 5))
 (segment (start 132.714 128.522) (end 132.714 128.873) (width 0.25) (layer F.Cu) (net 5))
 (segment (start 132.714 128.522) (end 132.714 128.873) (width 0.25) (layer F.Cu) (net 5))
 (segment (start 130.783 130.85) (end 130.533 131.1) (width 0.25) (layer F.Cu) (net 5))
 (segment (start 130.533 131.1) (end 129.109 131.1) (width 0.25) (layer F.Cu) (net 5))
 (segment (start 125.199 137.85) (end 125.199 135.01) (width 0.25) (layer B.Cu) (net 5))
 (segment (start 125.199 135.01) (end 129.109 131.1) (width 0.25) (layer B.Cu) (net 5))
 (via (at 129.109 131.1) (size 0.6) (layers F.Cu B.Cu) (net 5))
 (segment (start 112.395 115.57) (end 116.447 115.57) (width 0.25) (layer B.Cu) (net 9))
 (segment (start 116.447 115.57) (end 124.091 123.213) (width 0.25) (layer B.Cu) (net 9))
 (segment (start 124.091 123.213) (end 124.391 123.513) (width 0.25) (layer B.Cu) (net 9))
 (segment (start 128.714 128.522) (end 128.714 127.784) (width 0.25) (layer F.Cu) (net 9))
 (segment (start 128.714 127.784) (end 124.443 123.513) (width 0.25) (layer F.Cu) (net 9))
 (segment (start 124.443 123.513) (end 124.391 123.513) (width 0.25) (layer F.Cu) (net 9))
 (via (at 124.391 123.513) (size 0.6) (layers F.Cu B.Cu) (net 9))
 (segment (start 126.714 128.522) (end 126.714 126.772) (width 0.25) (layer F.Cu) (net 10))
 (segment (start 126.714 126.772) (end 124.021 124.079) (width 0.25) (layer F.Cu) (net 10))
 (segment (start 124.021 124.079) (end 123.571 124.079) (width 0.25) (layer F.Cu) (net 10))
 (segment (start 112.395 118.11) (end 117.602 118.11) (width 0.25) (layer B.Cu) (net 10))
 (segment (start 117.602 118.11) (end 123.571 124.079) (width 0.25) (layer B.Cu) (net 10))
 (via (at 123.571 124.079) (size 0.6) (layers F.Cu B.Cu) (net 10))
 (segment (start 122.714 128.522) (end 122.714 126.772) (width 0.25) (layer F.Cu) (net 12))
 (segment (start 122.714 126.772) (end 122.053 126.111) (width 0.25) (layer F.Cu) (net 12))
 (segment (start 122.053 126.111) (end 121.793 126.111) (width 0.25) (layer F.Cu) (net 12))
 (segment (start 121.793 126.111) (end 119.907 126.111) (width 0.25) (layer B.Cu) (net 12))
 (segment (start 119.907 126.111) (end 116.986 123.19) (width 0.25) (layer B.Cu) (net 12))
 (segment (start 116.986 123.19) (end 112.395 123.19) (width 0.25) (layer B.Cu) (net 12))
 (segment (start 128.859 132.15) (end 128.459 132.15) (width 0.25) (layer F.Cu) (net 12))
 (segment (start 128.459 132.15) (end 126.656 130.347) (width 0.25) (layer F.Cu) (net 12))
 (segment (start 126.656 130.347) (end 123.801 130.347) (width 0.25) (layer F.Cu) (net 12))
 (segment (start 123.801 130.347) (end 122.714 129.26) (width 0.25) (layer F.Cu) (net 12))
 (segment (start 122.714 129.26) (end 122.714 128.522) (width 0.25) (layer F.Cu) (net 12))
 (via (at 121.793 126.111) (size 0.6) (layers F.Cu B.Cu) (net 12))
 (segment (start 120.714 128.522) (end 120.714 126.772) (width 0.25) (layer F.Cu) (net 13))
 (segment (start 120.714 126.772) (end 120.399 126.457) (width 0.25) (layer F.Cu) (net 13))
 (segment (start 120.399 126.457) (end 119.328 126.457) (width 0.25) (layer F.Cu) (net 13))
 (segment (start 119.328 126.457) (end 113.122 126.457) (width 0.25) (layer B.Cu) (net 13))
 (segment (start 113.122 126.457) (end 112.395 125.73) (width 0.25) (layer B.Cu) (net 13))
 (segment (start 125.859 132.15) (end 124.759 132.15) (width 0.25) (layer F.Cu) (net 13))
 (segment (start 124.759 132.15) (end 122.956 130.347) (width 0.25) (layer F.Cu) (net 13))
 (segment (start 122.956 130.347) (end 121.801 130.347) (width 0.25) (layer F.Cu) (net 13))
 (segment (start 121.801 130.347) (end 120.714 129.26) (width 0.25) (layer F.Cu) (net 13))
 (segment (start 120.714 129.26) (end 120.714 128.522) (width 0.25) (layer F.Cu) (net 13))
 (via (at 119.328 126.457) (size 0.6) (layers F.Cu B.Cu) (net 13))
 (segment (start 120.714 112.522) (end 120.714 113.26) (width 0.25) (layer F.Cu) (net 14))
 (segment (start 120.714 113.26) (end 113.736 120.238) (width 0.25) (layer F.Cu) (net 14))
 (segment (start 113.736 120.238) (end 113.736 123.682) (width 0.25) (layer F.Cu) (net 14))
 (segment (start 113.736 123.682) (end 112.877 124.541) (width 0.25) (layer F.Cu) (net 14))
 (segment (start 112.877 124.541) (end 111.75 124.541) (width 0.25) (layer F.Cu) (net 14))
 (segment (start 111.75 124.541) (end 111.054 125.238) (width 0.25) (layer F.Cu) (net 14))
 (segment (start 111.054 125.238) (end 111.054 127.081) (width 0.25) (layer F.Cu) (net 14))
 (segment (start 111.054 127.081) (end 112.243 128.27) (width 0.25) (layer F.Cu) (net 14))
 (segment (start 112.243 128.27) (end 112.395 128.27) (width 0.25) (layer F.Cu) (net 14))
 (segment (start 122.714 112.522) (end 122.714 115.341) (width 0.25) (layer F.Cu) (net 15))
 (segment (start 122.714 115.341) (end 113.736 124.319) (width 0.25) (layer F.Cu) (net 15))
 (segment (start 113.736 124.319) (end 113.736 129.621) (width 0.25) (layer F.Cu) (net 15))
 (segment (start 113.736 129.621) (end 112.547 130.81) (width 0.25) (layer F.Cu) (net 15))
 (segment (start 112.547 130.81) (end 112.395 130.81) (width 0.25) (layer F.Cu) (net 15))
 (segment (start 124.714 112.522) (end 124.714 113.26) (width 0.25) (layer F.Cu) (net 16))
 (segment (start 124.714 113.26) (end 123.702 114.272) (width 0.25) (layer F.Cu) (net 16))
 (segment (start 123.702 114.272) (end 123.702 114.989) (width 0.25) (layer F.Cu) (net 16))
 (segment (start 123.702 114.989) (end 114.186 124.505) (width 0.25) (layer F.Cu) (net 16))
 (segment (start 114.186 124.505) (end 114.186 131.711) (width 0.25) (layer F.Cu) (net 16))
 (segment (start 114.186 131.711) (end 112.547 133.35) (width 0.25) (layer F.Cu) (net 16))
 (segment (start 112.547 133.35) (end 112.395 133.35) (width 0.25) (layer F.Cu) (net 16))
 (segment (start 126.714 112.522) (end 126.714 113.26) (width 0.25) (layer F.Cu) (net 17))
 (segment (start 126.714 113.26) (end 116.913 123.061) (width 0.25) (layer F.Cu) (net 17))
 (segment (start 116.913 123.061) (end 116.267 123.061) (width 0.25) (layer F.Cu) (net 17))
 (segment (start 116.267 123.061) (end 114.636 124.692) (width 0.25) (layer F.Cu) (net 17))
 (segment (start 114.636 124.692) (end 114.636 133.801) (width 0.25) (layer F.Cu) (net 17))
 (segment (start 114.636 133.801) (end 112.547 135.89) (width 0.25) (layer F.Cu) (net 17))
 (segment (start 112.547 135.89) (end 112.395 135.89) (width 0.25) (layer F.Cu) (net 17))
 (segment (start 130.714 112.522) (end 130.714 113.26) (width 0.25) (layer F.Cu) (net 18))
 (segment (start 130.714 113.26) (end 129.702 114.272) (width 0.25) (layer F.Cu) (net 18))
 (segment (start 129.702 114.272) (end 129.702 114.501) (width 0.25) (layer F.Cu) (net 18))
 (segment (start 129.702 114.501) (end 126.723 117.48) (width 0.25) (layer F.Cu) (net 18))
 (segment (start 126.723 117.48) (end 126.494 117.48) (width 0.25) (layer F.Cu) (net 18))
 (segment (start 126.494 117.48) (end 119.546 124.428) (width 0.25) (layer F.Cu) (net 18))
 (segment (start 119.546 124.428) (end 115.536 124.428) (width 0.25) (layer F.Cu) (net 18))
 (segment (start 115.536 124.428) (end 115.086 124.878) (width 0.25) (layer F.Cu) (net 18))
 (segment (start 115.086 124.878) (end 115.086 135.891) (width 0.25) (layer F.Cu) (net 18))
 (segment (start 115.086 135.891) (end 112.547 138.43) (width 0.25) (layer F.Cu) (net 18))
 (segment (start 112.547 138.43) (end 112.395 138.43) (width 0.25) (layer F.Cu) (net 18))
 (segment (start 139.865 107.173) (end 139.8649 107.173) (width 0.25) (layer F.Cu) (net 2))
 (segment (start 139.8649 107.173) (end 139.8499 107.188) (width 0.25) (layer F.Cu) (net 2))
 (segment (start 139.865 107.173) (end 139.85 107.188) (width 0.25) (layer F.Cu) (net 2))
 (segment (start 139.88 104.648) (end 139.88 107.158) (width 0.25) (layer F.Cu) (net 2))
 (segment (start 139.88 107.158) (end 139.865 107.173) (width 0.25) (layer F.Cu) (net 2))
 (segment (start 132.059 132.15) (end 131.859 132.15) (width 0.25) (layer F.Cu) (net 19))
 (segment (start 132.521 124.438) (end 132.521 126.054) (width 0.25) (layer F.Cu) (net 19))
 (segment (start 132.521 126.054) (end 133.801 127.334) (width 0.25) (layer F.Cu) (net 19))
 (segment (start 133.801 127.334) (end 133.801 130.608) (width 0.25) (layer F.Cu) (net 19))
 (segment (start 133.801 130.608) (end 132.259 132.15) (width 0.25) (layer F.Cu) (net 19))
 (segment (start 132.259 132.15) (end 132.059 132.15) (width 0.25) (layer F.Cu) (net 19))
 (segment (start 132.059 132.588) (end 132.194 132.588) (width 0.5) (layer F.Cu) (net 19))
 (segment (start 131.244 132.588) (end 132.059 132.588) (width 0.5) (layer F.Cu) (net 19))
 (segment (start 132.059 132.15) (end 132.059 132.588) (width 0.25) (layer F.Cu) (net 19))
 (segment (start 128.714 112.522) (end 128.714 111.784) (width 0.5) (layer F.Cu) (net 19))
 (segment (start 128.714 112.522) (end 128.714 113.602) (width 0.5) (layer F.Cu) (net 19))
 (segment (start 128.714 112.522) (end 128.714 113.26) (width 0.25) (layer F.Cu) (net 19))
 (segment (start 128.714 113.26) (end 125.859 116.115) (width 0.25) (layer F.Cu) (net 19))
 (segment (start 125.859 116.115) (end 125.859 116.6) (width 0.25) (layer F.Cu) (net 19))
 (segment (start 125.859 116.6) (end 125.859 117.775) (width 0.25) (layer B.Cu) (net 19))
 (segment (start 125.859 117.775) (end 132.521 124.438) (width 0.25) (layer B.Cu) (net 19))
 (via (at 125.859 116.6) (size 0.6) (layers F.Cu B.Cu) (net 19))
 (via (at 132.521 124.438) (size 0.6) (layers F.Cu B.Cu) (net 19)))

